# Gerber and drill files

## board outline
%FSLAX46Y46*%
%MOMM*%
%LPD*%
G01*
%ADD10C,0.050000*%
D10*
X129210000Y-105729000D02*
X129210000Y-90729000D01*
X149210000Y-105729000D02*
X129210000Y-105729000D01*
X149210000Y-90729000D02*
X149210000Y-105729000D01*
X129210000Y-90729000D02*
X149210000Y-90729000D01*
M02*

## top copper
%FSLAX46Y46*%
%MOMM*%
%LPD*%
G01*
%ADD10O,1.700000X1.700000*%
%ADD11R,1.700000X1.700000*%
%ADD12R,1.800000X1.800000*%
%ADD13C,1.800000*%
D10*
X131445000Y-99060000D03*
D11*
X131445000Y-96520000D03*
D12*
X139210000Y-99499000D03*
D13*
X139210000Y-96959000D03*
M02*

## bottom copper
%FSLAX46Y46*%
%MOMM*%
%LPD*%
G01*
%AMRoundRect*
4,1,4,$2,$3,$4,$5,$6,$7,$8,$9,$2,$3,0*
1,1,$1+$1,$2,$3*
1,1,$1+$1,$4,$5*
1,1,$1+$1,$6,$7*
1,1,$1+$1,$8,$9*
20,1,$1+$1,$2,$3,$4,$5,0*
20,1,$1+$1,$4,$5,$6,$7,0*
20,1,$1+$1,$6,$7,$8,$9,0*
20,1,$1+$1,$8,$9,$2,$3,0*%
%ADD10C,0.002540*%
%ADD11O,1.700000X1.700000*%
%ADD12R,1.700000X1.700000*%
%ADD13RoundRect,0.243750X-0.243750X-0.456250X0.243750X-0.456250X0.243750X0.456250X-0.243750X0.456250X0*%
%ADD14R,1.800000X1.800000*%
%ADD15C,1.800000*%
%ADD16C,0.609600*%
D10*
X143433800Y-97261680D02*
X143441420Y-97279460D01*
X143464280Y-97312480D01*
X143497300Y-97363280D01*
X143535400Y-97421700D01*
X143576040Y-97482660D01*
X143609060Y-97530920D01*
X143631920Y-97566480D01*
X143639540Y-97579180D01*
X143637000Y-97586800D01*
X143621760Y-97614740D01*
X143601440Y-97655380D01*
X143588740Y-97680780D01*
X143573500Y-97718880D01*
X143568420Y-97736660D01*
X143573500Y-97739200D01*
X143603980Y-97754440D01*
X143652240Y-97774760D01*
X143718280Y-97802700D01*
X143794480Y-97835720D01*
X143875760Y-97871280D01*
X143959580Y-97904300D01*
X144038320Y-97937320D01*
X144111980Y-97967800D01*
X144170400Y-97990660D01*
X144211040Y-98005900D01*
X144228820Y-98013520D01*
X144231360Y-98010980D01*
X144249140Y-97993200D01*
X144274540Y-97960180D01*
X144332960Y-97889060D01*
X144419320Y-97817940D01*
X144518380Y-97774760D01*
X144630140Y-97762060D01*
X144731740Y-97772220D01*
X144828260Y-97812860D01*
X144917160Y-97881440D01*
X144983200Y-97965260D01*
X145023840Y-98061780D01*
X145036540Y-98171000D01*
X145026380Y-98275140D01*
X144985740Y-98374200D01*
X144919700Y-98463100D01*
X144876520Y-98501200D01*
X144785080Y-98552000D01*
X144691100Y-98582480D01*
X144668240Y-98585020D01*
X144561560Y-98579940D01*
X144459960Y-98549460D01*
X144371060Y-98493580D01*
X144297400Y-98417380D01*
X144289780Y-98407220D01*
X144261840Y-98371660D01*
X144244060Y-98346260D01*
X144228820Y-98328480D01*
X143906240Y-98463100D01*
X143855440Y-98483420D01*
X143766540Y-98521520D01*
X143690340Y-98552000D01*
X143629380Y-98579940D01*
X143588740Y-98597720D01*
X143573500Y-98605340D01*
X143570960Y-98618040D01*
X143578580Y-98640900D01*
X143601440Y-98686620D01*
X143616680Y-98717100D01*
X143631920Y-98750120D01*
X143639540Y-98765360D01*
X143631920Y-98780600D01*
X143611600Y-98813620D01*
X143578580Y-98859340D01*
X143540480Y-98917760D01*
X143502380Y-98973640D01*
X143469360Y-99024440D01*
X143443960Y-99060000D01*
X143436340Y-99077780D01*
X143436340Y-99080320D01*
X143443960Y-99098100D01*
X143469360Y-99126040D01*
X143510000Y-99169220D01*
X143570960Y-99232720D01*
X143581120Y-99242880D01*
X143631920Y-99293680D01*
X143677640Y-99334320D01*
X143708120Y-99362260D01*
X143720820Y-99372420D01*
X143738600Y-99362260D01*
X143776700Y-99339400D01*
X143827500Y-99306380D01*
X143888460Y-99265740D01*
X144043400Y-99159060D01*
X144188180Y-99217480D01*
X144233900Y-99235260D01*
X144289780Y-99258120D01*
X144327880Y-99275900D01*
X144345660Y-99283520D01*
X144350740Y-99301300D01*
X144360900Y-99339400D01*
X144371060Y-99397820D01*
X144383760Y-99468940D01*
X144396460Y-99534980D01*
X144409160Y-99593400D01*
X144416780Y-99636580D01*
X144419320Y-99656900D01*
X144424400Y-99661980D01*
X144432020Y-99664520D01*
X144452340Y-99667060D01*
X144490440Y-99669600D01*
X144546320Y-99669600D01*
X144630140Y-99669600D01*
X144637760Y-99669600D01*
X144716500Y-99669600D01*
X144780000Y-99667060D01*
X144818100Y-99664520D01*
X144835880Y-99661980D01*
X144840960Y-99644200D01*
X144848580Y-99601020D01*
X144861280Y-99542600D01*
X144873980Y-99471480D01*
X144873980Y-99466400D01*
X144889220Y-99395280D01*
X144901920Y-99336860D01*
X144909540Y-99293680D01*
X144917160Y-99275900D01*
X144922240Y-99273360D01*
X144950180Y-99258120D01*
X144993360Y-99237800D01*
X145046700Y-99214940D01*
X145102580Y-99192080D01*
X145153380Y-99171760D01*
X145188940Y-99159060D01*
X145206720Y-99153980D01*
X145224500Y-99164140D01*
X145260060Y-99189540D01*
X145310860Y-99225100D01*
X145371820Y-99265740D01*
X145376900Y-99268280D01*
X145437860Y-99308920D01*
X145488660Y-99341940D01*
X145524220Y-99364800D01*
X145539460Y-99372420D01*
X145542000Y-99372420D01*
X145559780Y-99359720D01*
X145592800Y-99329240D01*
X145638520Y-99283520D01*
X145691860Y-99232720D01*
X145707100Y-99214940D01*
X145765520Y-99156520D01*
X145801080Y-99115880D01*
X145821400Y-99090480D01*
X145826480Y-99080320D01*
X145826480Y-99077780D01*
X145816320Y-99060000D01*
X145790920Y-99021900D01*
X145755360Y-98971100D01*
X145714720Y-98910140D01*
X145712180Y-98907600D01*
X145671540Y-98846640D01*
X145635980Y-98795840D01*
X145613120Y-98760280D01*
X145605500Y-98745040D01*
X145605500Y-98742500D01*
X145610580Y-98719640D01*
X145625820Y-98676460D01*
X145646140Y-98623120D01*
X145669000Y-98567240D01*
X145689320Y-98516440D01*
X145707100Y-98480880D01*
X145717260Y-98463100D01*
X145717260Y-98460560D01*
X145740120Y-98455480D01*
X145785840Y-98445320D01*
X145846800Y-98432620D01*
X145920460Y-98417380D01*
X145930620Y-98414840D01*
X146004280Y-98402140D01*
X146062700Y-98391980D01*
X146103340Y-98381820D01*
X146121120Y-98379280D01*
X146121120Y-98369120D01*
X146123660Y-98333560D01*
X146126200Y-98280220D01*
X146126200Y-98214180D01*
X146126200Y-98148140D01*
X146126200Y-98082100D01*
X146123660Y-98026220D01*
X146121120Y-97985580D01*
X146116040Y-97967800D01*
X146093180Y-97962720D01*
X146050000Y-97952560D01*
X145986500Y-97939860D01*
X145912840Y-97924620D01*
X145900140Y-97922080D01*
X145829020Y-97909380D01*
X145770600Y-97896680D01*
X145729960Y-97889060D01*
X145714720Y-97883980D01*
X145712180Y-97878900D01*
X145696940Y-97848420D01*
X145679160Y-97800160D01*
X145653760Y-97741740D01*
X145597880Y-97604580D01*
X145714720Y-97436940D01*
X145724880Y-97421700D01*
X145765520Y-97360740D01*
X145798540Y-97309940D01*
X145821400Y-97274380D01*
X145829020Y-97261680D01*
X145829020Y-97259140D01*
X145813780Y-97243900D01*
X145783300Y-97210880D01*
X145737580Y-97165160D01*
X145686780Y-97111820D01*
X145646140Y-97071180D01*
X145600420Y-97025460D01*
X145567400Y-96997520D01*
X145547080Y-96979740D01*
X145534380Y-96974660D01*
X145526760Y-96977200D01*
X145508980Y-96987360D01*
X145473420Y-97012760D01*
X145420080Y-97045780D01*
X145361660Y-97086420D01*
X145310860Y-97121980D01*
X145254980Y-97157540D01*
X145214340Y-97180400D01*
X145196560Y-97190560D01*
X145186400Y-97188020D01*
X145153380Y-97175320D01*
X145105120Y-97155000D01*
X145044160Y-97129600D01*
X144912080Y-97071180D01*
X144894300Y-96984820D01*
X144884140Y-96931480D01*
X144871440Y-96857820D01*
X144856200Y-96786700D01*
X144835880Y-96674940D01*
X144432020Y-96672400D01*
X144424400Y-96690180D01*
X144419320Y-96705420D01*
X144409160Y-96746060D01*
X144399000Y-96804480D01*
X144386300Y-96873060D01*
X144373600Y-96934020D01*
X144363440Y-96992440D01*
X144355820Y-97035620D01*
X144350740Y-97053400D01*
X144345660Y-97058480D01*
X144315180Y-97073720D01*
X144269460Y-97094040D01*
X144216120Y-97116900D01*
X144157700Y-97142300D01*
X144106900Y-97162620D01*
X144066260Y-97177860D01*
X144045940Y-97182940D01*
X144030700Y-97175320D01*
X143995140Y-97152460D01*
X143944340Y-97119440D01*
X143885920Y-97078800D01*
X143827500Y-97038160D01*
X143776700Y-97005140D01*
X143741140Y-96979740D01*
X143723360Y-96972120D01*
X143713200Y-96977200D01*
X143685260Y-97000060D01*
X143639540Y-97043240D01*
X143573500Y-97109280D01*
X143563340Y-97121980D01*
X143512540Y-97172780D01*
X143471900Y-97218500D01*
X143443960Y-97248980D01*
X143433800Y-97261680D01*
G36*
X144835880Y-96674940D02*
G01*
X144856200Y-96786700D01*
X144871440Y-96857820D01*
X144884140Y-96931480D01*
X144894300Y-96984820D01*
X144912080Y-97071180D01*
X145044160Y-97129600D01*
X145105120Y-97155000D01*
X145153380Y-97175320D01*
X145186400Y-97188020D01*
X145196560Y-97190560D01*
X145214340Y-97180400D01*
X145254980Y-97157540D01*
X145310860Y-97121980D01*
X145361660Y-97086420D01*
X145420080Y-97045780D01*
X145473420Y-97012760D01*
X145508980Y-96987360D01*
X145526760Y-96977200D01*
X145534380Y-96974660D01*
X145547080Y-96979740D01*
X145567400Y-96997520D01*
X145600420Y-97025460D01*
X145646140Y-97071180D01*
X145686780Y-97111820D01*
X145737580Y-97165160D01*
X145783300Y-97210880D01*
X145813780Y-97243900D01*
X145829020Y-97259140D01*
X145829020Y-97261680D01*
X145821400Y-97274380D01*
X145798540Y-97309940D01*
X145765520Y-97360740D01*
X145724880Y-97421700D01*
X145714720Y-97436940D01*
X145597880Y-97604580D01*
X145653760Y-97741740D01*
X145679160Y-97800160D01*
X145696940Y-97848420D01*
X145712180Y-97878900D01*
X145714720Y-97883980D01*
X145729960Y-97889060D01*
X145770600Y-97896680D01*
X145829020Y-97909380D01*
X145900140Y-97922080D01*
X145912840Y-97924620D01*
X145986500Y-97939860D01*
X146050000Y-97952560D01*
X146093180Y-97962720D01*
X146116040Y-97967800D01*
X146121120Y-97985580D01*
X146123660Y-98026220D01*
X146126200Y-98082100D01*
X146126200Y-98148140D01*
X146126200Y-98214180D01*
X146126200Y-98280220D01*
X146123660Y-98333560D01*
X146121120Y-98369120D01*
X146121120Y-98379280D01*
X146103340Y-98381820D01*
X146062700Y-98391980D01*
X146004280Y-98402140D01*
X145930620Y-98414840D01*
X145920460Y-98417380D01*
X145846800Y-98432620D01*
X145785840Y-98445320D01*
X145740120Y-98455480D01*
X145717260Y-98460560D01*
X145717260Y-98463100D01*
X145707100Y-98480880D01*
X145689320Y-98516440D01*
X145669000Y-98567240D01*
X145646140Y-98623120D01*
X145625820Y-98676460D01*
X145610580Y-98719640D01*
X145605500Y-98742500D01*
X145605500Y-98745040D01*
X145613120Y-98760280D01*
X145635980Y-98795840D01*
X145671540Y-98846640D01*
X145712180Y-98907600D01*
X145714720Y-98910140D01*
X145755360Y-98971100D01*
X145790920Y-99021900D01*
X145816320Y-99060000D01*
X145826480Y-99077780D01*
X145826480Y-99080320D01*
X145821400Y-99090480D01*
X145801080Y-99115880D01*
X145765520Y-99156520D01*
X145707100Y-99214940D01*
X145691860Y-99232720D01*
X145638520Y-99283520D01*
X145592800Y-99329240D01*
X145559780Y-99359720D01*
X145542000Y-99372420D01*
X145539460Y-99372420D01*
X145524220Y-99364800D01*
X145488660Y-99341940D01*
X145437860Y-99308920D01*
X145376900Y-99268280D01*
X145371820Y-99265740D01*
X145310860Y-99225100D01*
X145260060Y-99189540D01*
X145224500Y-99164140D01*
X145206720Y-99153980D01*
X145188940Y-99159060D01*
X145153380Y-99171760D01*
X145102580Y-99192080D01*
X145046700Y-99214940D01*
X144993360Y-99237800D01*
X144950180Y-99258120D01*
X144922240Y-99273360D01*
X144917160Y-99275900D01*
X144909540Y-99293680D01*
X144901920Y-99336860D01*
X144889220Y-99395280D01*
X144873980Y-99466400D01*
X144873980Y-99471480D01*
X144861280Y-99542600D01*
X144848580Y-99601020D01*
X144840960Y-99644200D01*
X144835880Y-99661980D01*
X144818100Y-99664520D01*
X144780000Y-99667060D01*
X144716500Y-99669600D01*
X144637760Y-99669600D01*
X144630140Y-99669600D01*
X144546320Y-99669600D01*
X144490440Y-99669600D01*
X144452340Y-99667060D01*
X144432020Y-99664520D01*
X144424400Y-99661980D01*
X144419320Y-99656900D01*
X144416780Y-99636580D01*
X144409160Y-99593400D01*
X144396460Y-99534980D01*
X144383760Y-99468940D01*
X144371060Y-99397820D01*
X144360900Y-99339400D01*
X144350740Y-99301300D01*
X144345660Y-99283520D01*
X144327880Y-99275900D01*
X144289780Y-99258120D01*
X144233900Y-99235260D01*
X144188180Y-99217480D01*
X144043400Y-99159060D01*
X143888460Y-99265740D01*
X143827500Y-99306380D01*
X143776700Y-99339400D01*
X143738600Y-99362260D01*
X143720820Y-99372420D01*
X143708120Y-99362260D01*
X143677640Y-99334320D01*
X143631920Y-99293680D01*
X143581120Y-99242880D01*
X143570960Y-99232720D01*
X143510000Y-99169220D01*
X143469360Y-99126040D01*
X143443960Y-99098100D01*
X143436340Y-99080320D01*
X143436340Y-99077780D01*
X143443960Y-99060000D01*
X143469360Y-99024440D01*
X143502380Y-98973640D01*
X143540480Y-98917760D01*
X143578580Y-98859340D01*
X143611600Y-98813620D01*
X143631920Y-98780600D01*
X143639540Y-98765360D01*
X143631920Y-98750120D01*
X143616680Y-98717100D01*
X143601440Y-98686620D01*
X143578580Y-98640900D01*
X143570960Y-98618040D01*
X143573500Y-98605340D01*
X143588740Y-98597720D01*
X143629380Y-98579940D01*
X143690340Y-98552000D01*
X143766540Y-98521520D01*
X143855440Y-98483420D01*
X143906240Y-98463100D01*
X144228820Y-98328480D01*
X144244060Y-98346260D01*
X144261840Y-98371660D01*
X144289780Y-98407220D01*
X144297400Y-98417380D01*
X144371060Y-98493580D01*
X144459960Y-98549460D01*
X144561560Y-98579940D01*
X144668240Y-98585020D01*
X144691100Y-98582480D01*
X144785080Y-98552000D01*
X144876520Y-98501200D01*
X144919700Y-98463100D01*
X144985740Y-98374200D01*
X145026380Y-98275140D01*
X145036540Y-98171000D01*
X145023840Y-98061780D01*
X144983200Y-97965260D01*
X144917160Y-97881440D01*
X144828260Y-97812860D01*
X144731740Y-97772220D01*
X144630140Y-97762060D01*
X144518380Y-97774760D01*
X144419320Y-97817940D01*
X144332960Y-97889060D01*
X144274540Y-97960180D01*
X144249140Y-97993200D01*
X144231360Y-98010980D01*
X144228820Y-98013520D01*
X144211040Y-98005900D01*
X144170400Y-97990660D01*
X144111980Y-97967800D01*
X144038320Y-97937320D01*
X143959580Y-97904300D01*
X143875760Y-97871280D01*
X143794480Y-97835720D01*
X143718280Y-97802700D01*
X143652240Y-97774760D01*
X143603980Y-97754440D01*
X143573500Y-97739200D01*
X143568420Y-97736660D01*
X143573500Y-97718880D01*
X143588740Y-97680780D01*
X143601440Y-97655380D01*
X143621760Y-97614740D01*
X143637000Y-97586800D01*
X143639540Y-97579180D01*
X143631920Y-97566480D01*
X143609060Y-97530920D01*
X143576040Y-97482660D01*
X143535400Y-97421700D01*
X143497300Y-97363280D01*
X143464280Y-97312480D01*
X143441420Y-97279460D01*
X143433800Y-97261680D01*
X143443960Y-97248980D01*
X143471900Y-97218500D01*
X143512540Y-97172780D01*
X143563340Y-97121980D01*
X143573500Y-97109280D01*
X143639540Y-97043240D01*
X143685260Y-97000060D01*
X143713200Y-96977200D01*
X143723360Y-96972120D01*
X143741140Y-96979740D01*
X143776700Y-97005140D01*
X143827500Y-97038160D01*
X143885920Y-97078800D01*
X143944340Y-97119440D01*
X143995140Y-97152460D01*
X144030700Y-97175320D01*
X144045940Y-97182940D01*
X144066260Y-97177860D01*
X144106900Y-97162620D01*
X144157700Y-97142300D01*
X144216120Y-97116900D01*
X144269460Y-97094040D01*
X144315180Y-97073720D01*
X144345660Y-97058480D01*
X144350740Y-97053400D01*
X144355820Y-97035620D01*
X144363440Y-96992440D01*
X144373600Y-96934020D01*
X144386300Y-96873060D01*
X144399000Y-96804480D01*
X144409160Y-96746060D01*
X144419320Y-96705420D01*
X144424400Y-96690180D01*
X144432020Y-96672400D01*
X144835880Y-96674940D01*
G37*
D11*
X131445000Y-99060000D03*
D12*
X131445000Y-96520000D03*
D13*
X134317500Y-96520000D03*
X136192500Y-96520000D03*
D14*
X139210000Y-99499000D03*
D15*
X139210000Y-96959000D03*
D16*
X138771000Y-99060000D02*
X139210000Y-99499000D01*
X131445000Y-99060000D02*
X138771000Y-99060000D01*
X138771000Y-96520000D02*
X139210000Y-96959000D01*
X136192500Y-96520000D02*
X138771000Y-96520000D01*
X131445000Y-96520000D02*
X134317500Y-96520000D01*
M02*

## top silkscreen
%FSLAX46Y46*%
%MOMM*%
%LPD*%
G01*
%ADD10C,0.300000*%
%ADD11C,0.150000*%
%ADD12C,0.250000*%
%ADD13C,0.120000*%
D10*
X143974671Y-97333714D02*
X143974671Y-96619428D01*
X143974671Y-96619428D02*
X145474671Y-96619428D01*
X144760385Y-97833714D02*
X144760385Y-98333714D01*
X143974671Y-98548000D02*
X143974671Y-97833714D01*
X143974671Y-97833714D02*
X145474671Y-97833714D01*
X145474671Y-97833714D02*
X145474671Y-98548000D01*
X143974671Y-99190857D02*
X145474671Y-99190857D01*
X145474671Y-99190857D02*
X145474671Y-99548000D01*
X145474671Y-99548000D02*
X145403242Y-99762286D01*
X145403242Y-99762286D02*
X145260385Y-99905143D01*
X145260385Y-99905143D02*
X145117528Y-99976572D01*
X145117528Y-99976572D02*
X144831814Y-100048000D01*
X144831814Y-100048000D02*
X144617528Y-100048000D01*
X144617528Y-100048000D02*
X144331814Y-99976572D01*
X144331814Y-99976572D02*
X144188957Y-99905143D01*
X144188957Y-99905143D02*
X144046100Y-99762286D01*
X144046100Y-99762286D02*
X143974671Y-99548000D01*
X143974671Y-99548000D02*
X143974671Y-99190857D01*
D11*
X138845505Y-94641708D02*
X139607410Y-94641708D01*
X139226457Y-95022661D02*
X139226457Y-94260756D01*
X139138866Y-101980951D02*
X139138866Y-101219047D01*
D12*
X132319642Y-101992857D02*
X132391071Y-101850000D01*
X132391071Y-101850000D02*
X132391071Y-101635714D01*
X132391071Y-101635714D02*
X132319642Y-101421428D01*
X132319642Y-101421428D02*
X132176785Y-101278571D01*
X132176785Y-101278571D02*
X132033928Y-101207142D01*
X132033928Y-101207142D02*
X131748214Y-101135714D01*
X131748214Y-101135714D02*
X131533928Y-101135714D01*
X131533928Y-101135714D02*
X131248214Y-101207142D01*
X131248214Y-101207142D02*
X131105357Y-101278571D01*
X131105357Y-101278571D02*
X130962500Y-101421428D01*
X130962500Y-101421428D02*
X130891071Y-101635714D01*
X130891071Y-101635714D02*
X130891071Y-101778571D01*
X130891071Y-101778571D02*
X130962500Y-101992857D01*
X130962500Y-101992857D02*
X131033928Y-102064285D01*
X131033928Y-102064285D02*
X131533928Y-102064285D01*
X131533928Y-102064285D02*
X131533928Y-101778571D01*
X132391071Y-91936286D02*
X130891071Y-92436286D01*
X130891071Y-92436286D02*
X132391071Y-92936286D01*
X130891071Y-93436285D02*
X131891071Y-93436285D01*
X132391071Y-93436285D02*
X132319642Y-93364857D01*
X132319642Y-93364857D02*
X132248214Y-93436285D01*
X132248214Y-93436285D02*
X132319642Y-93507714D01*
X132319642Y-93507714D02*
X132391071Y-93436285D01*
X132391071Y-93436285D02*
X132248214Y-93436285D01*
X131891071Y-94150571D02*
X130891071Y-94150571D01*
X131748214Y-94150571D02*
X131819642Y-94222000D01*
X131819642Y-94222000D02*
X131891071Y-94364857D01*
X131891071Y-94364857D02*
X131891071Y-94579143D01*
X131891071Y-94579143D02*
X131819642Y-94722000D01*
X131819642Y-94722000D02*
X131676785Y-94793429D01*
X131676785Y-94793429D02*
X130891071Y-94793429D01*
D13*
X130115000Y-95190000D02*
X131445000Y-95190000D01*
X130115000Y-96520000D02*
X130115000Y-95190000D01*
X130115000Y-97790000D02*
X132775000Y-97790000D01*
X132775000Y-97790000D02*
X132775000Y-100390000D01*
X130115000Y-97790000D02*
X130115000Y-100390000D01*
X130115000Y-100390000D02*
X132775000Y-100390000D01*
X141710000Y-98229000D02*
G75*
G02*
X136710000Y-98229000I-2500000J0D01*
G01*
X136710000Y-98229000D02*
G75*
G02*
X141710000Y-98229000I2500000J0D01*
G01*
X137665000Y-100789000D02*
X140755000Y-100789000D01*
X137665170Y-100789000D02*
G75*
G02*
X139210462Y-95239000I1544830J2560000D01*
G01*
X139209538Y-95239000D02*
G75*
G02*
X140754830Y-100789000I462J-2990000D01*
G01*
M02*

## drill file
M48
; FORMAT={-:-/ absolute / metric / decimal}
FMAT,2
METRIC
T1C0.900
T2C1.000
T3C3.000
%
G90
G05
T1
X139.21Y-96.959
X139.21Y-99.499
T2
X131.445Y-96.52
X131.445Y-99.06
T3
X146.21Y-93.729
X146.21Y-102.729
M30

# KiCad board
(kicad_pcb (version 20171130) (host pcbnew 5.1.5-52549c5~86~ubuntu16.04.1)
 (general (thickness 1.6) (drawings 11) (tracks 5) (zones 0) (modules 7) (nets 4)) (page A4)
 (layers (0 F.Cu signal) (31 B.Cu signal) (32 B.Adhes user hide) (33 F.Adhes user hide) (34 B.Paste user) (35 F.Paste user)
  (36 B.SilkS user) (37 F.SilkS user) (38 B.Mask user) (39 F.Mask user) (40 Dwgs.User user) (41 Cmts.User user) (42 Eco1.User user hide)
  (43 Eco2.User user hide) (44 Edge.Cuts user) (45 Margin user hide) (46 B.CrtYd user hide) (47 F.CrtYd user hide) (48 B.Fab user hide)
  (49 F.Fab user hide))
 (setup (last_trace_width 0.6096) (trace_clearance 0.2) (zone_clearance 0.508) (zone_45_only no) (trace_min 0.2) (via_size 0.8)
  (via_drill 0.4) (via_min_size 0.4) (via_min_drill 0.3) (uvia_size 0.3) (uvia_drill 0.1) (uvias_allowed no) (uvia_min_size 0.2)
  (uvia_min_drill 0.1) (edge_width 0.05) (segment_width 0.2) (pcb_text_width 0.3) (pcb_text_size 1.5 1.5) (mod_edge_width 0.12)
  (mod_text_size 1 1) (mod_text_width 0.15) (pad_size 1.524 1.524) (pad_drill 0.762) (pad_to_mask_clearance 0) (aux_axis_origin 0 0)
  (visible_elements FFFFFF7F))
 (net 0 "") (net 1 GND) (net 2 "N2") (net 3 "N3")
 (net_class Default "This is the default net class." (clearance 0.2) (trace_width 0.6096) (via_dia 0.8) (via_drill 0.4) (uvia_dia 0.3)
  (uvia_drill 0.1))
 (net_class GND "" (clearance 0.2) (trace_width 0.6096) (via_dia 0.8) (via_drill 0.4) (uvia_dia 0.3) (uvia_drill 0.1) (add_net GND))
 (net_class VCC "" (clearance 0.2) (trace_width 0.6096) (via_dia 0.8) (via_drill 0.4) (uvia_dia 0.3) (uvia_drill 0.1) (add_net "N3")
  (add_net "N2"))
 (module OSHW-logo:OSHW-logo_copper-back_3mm (layer B.Cu) (at 144.78 98.171 90)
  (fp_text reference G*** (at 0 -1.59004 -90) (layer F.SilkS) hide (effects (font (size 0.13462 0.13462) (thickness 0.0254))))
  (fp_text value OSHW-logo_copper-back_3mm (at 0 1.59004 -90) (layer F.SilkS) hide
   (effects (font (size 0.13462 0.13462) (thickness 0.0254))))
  (fp_poly
   (pts (xy 0.90932 -1.3462) (xy 0.89154 -1.33858) (xy 0.85852 -1.31572) (xy 0.80772 -1.2827) (xy 0.7493 -1.2446) (xy 0.68834 -1.20396)
    (xy 0.64008 -1.17094) (xy 0.60452 -1.14808) (xy 0.59182 -1.14046) (xy 0.5842 -1.143) (xy 0.55626 -1.15824) (xy 0.51562 -1.17856)
    (xy 0.49022 -1.19126) (xy 0.45212 -1.2065) (xy 0.43434 -1.21158) (xy 0.4318 -1.2065) (xy 0.41656 -1.17602) (xy 0.39624 -1.12776)
    (xy 0.3683 -1.06172) (xy 0.33528 -0.98552) (xy 0.29972 -0.90424) (xy 0.2667 -0.82042) (xy 0.23368 -0.74168) (xy 0.2032 -0.66802)
    (xy 0.18034 -0.6096) (xy 0.1651 -0.56896) (xy 0.15748 -0.55118) (xy 0.16002 -0.54864) (xy 0.1778 -0.53086) (xy 0.21082 -0.50546)
    (xy 0.28194 -0.44704) (xy 0.35306 -0.36068) (xy 0.39624 -0.26162) (xy 0.40894 -0.14986) (xy 0.39878 -0.04826) (xy 0.35814 0.04826)
    (xy 0.28956 0.13716) (xy 0.20574 0.2032) (xy 0.10922 0.24384) (xy 0 0.25654) (xy -0.10414 0.24638) (xy -0.2032 0.20574)
    (xy -0.2921 0.1397) (xy -0.3302 0.09652) (xy -0.381 0.00508) (xy -0.41148 -0.0889) (xy -0.41402 -0.11176) (xy -0.40894 -0.21844)
    (xy -0.37846 -0.32004) (xy -0.32258 -0.40894) (xy -0.24638 -0.4826) (xy -0.23622 -0.49022) (xy -0.20066 -0.51816) (xy -0.17526 -0.53594)
    (xy -0.15748 -0.55118) (xy -0.2921 -0.87376) (xy -0.31242 -0.92456) (xy -0.35052 -1.01346) (xy -0.381 -1.08966) (xy -0.40894 -1.15062)
    (xy -0.42672 -1.19126) (xy -0.43434 -1.2065) (xy -0.44704 -1.20904) (xy -0.4699 -1.20142) (xy -0.51562 -1.17856) (xy -0.5461 -1.16332)
    (xy -0.57912 -1.14808) (xy -0.59436 -1.14046) (xy -0.6096 -1.14808) (xy -0.64262 -1.1684) (xy -0.68834 -1.20142) (xy -0.74676 -1.23952)
    (xy -0.80264 -1.27762) (xy -0.85344 -1.31064) (xy -0.889 -1.33604) (xy -0.90678 -1.34366) (xy -0.90932 -1.34366) (xy -0.9271 -1.33604)
    (xy -0.95504 -1.31064) (xy -0.99822 -1.27) (xy -1.06172 -1.20904) (xy -1.07188 -1.19888) (xy -1.12268 -1.14808) (xy -1.16332 -1.10236)
    (xy -1.19126 -1.07188) (xy -1.20142 -1.05918) (xy -1.19126 -1.0414) (xy -1.1684 -1.0033) (xy -1.13538 -0.9525) (xy -1.09474 -0.89154)
    (xy -0.98806 -0.7366) (xy -1.04648 -0.59182) (xy -1.06426 -0.5461) (xy -1.08712 -0.49022) (xy -1.1049 -0.45212) (xy -1.11252 -0.43434)
    (xy -1.1303 -0.42926) (xy -1.1684 -0.4191) (xy -1.22682 -0.40894) (xy -1.29794 -0.39624) (xy -1.36398 -0.38354) (xy -1.4224 -0.37084)
    (xy -1.46558 -0.36322) (xy -1.4859 -0.36068) (xy -1.49098 -0.3556) (xy -1.49352 -0.34798) (xy -1.49606 -0.32766) (xy -1.4986 -0.28956)
    (xy -1.4986 -0.23368) (xy -1.4986 -0.14986) (xy -1.4986 -0.14224) (xy -1.4986 -0.0635) (xy -1.49606 0) (xy -1.49352 0.0381)
    (xy -1.49098 0.05588) (xy -1.4732 0.06096) (xy -1.43002 0.06858) (xy -1.3716 0.08128) (xy -1.30048 0.09398) (xy -1.2954 0.09398)
    (xy -1.22428 0.10922) (xy -1.16586 0.12192) (xy -1.12268 0.12954) (xy -1.1049 0.13716) (xy -1.10236 0.14224) (xy -1.08712 0.17018)
    (xy -1.0668 0.21336) (xy -1.04394 0.2667) (xy -1.02108 0.32258) (xy -1.00076 0.37338) (xy -0.98806 0.40894) (xy -0.98298 0.42672)
    (xy -0.99314 0.4445) (xy -1.01854 0.48006) (xy -1.0541 0.53086) (xy -1.09474 0.59182) (xy -1.09728 0.5969) (xy -1.13792 0.65786)
    (xy -1.17094 0.70866) (xy -1.1938 0.74422) (xy -1.20142 0.75946) (xy -1.20142 0.762) (xy -1.18872 0.77978) (xy -1.15824 0.8128)
    (xy -1.11252 0.85852) (xy -1.06172 0.91186) (xy -1.04394 0.9271) (xy -0.98552 0.98552) (xy -0.94488 1.02108) (xy -0.91948 1.0414)
    (xy -0.90932 1.04648) (xy -0.90678 1.04648) (xy -0.889 1.03632) (xy -0.8509 1.01092) (xy -0.8001 0.97536) (xy -0.73914 0.93472)
    (xy -0.7366 0.93218) (xy -0.67564 0.89154) (xy -0.62484 0.85598) (xy -0.58928 0.83312) (xy -0.57404 0.8255) (xy -0.5715 0.8255)
    (xy -0.54864 0.83058) (xy -0.50546 0.84582) (xy -0.45212 0.86614) (xy -0.39624 0.889) (xy -0.34544 0.90932) (xy -0.30988 0.9271)
    (xy -0.2921 0.93726) (xy -0.28956 0.93726) (xy -0.28448 0.96012) (xy -0.27432 1.00584) (xy -0.26162 1.0668) (xy -0.24638 1.14046)
    (xy -0.24384 1.15062) (xy -0.23114 1.22428) (xy -0.22098 1.2827) (xy -0.21082 1.32334) (xy -0.20828 1.34112) (xy -0.19812 1.34112)
    (xy -0.16256 1.34366) (xy -0.10922 1.3462) (xy -0.04318 1.3462) (xy 0.02286 1.3462) (xy 0.0889 1.3462) (xy 0.14478 1.34366)
    (xy 0.18542 1.34112) (xy 0.2032 1.33604) (xy 0.20828 1.31318) (xy 0.21844 1.27) (xy 0.23114 1.2065) (xy 0.24638 1.13284)
    (xy 0.24892 1.12014) (xy 0.26162 1.04902) (xy 0.27432 0.9906) (xy 0.28194 0.94996) (xy 0.28702 0.93472) (xy 0.2921 0.93218)
    (xy 0.32258 0.91694) (xy 0.37084 0.89916) (xy 0.42926 0.87376) (xy 0.56642 0.81788) (xy 0.73406 0.93472) (xy 0.7493 0.94488)
    (xy 0.81026 0.98552) (xy 0.86106 1.01854) (xy 0.89662 1.0414) (xy 0.90932 1.04902) (xy 0.91186 1.04902) (xy 0.9271 1.03378)
    (xy 0.96012 1.0033) (xy 1.00584 0.95758) (xy 1.05918 0.90678) (xy 1.09982 0.86614) (xy 1.14554 0.82042) (xy 1.17348 0.7874)
    (xy 1.19126 0.76708) (xy 1.19634 0.75438) (xy 1.1938 0.74676) (xy 1.18364 0.72898) (xy 1.15824 0.69342) (xy 1.12522 0.64008)
    (xy 1.08458 0.58166) (xy 1.04902 0.53086) (xy 1.01346 0.47498) (xy 0.9906 0.43434) (xy 0.98044 0.41656) (xy 0.98298 0.4064)
    (xy 0.99568 0.37338) (xy 1.016 0.32512) (xy 1.0414 0.26416) (xy 1.09982 0.13208) (xy 1.18618 0.1143) (xy 1.23952 0.10414)
    (xy 1.31318 0.09144) (xy 1.3843 0.0762) (xy 1.49606 0.05588) (xy 1.4986 -0.34798) (xy 1.48082 -0.3556) (xy 1.46558 -0.36068)
    (xy 1.42494 -0.37084) (xy 1.36652 -0.381) (xy 1.29794 -0.3937) (xy 1.23698 -0.4064) (xy 1.17856 -0.41656) (xy 1.13538 -0.42418)
    (xy 1.1176 -0.42926) (xy 1.11252 -0.43434) (xy 1.09728 -0.46482) (xy 1.07696 -0.51054) (xy 1.0541 -0.56388) (xy 1.0287 -0.6223)
    (xy 1.00838 -0.6731) (xy 0.99314 -0.71374) (xy 0.98806 -0.73406) (xy 0.99568 -0.7493) (xy 1.01854 -0.78486) (xy 1.05156 -0.83566)
    (xy 1.0922 -0.89408) (xy 1.13284 -0.9525) (xy 1.16586 -1.0033) (xy 1.19126 -1.03886) (xy 1.19888 -1.05664) (xy 1.1938 -1.0668)
    (xy 1.17094 -1.09474) (xy 1.12776 -1.14046) (xy 1.06172 -1.2065) (xy 1.04902 -1.21666) (xy 0.99822 -1.26746) (xy 0.9525 -1.3081)
    (xy 0.92202 -1.33604) (xy 0.90932 -1.3462))
   (layer B.Cu) (width 0.00254)))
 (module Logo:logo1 (layer B.Cu) (at 142.24 98.425 90)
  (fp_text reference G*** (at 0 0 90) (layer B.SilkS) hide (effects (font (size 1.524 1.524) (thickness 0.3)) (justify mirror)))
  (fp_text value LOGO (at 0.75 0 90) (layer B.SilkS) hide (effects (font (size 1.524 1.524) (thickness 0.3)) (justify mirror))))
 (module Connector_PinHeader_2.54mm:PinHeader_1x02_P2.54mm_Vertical (layer F.Cu) (at 131.445 96.52)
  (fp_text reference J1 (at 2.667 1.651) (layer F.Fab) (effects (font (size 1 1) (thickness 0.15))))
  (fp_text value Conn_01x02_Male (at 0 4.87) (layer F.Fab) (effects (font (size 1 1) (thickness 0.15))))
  (fp_line (start -1.33 -1.33) (end 0 -1.33) (layer F.SilkS) (width 0.12))
  (fp_line (start -1.33 0) (end -1.33 -1.33) (layer F.SilkS) (width 0.12))
  (fp_line (start -1.33 1.27) (end 1.33 1.27) (layer F.SilkS) (width 0.12))
  (fp_line (start 1.33 1.27) (end 1.33 3.87) (layer F.SilkS) (width 0.12))
  (fp_line (start -1.33 1.27) (end -1.33 3.87) (layer F.SilkS) (width 0.12))
  (fp_line (start -1.33 3.87) (end 1.33 3.87) (layer F.SilkS) (width 0.12))
  (pad 2 thru_hole oval (at 0 2.54) (size 1.7 1.7) (drill 1) (layers *.Cu *.Mask) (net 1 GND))
  (pad 1 thru_hole rect (at 0 0) (size 1.7 1.7) (drill 1) (layers *.Cu *.Mask) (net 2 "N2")))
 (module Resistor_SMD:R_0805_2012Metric (layer B.Cu) (at 135.255 96.52)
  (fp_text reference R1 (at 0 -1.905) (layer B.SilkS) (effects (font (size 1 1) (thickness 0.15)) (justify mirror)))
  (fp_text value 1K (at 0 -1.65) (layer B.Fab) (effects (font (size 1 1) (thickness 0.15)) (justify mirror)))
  (pad 1 smd roundrect (at -0.9375 0) (size 0.975 1.4) (layers B.Cu B.Paste B.Mask) (roundrect_rratio 0.25) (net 2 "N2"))
  (pad 2 smd roundrect (at 0.9375 0) (size 0.975 1.4) (layers B.Cu B.Paste B.Mask) (roundrect_rratio 0.25) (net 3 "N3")))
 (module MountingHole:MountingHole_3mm (layer F.Cu) (at 146.21 93.729)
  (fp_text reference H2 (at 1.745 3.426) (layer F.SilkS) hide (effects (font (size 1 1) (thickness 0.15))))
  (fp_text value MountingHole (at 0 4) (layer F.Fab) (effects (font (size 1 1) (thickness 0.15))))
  (pad 1 np_thru_hole circle (at 0 0) (size 3 3) (drill 3) (layers *.Cu *.Mask)))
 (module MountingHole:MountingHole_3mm (layer F.Cu) (at 146.21 102.729)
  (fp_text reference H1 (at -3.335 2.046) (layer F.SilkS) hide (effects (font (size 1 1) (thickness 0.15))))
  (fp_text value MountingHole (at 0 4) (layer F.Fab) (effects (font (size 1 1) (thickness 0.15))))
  (pad 1 np_thru_hole circle (at 0 0) (size 3 3) (drill 3) (layers *.Cu *.Mask)))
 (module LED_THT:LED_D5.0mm (layer F.Cu) (at 139.21 99.499 90)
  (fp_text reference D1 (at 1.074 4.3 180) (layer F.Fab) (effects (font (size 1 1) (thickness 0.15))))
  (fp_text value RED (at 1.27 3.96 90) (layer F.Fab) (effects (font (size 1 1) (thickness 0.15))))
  (fp_circle (center 1.27 0) (end 3.77 0) (layer F.SilkS) (width 0.12))
  (fp_line (start -1.29 -1.545) (end -1.29 1.545) (layer F.SilkS) (width 0.12))
  (fp_arc (start 1.27 0) (end -1.29 -1.54483) (angle 148.9) (layer F.SilkS) (width 0.12))
  (fp_arc (start 1.27 0) (end -1.29 1.54483) (angle -148.9) (layer F.SilkS) (width 0.12))
  (pad 1 thru_hole rect (at 0 0 90) (size 1.8 1.8) (drill 0.9) (layers *.Cu *.Mask) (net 1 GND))
  (pad 2 thru_hole circle (at 2.54 0 90) (size 1.8 1.8) (drill 0.9) (layers *.Cu *.Mask) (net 3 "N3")))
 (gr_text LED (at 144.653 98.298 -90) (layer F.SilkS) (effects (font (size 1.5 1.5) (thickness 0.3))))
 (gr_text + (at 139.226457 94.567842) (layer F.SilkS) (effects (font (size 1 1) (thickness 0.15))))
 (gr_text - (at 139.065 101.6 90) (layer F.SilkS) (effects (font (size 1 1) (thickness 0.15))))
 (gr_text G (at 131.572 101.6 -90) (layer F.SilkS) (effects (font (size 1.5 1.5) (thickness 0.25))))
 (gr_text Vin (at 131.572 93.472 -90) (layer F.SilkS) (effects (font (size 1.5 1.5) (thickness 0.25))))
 (gr_line (start 129.21 105.729) (end 129.21 90.729) (layer Edge.Cuts) (width 0.05))
 (gr_line (start 149.21 105.729) (end 129.21 105.729) (layer Edge.Cuts) (width 0.05))
 (gr_line (start 149.21 90.729) (end 149.21 105.729) (layer Edge.Cuts) (width 0.05))
 (gr_line (start 129.21 90.729) (end 149.21 90.729) (layer Edge.Cuts) (width 0.05))
 (segment (start 138.771 99.06) (end 139.21 99.499) (width 0.6096) (layer B.Cu) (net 1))
 (segment (start 131.445 99.06) (end 138.771 99.06) (width 0.6096) (layer B.Cu) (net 1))
 (segment (start 138.771 96.52) (end 139.21 96.959) (width 0.6096) (layer B.Cu) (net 3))
 (segment (start 136.1925 96.52) (end 138.771 96.52) (width 0.6096) (layer B.Cu) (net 3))
 (segment (start 131.445 96.52) (end 134.3175 96.52) (width 0.6096) (layer B.Cu) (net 2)))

